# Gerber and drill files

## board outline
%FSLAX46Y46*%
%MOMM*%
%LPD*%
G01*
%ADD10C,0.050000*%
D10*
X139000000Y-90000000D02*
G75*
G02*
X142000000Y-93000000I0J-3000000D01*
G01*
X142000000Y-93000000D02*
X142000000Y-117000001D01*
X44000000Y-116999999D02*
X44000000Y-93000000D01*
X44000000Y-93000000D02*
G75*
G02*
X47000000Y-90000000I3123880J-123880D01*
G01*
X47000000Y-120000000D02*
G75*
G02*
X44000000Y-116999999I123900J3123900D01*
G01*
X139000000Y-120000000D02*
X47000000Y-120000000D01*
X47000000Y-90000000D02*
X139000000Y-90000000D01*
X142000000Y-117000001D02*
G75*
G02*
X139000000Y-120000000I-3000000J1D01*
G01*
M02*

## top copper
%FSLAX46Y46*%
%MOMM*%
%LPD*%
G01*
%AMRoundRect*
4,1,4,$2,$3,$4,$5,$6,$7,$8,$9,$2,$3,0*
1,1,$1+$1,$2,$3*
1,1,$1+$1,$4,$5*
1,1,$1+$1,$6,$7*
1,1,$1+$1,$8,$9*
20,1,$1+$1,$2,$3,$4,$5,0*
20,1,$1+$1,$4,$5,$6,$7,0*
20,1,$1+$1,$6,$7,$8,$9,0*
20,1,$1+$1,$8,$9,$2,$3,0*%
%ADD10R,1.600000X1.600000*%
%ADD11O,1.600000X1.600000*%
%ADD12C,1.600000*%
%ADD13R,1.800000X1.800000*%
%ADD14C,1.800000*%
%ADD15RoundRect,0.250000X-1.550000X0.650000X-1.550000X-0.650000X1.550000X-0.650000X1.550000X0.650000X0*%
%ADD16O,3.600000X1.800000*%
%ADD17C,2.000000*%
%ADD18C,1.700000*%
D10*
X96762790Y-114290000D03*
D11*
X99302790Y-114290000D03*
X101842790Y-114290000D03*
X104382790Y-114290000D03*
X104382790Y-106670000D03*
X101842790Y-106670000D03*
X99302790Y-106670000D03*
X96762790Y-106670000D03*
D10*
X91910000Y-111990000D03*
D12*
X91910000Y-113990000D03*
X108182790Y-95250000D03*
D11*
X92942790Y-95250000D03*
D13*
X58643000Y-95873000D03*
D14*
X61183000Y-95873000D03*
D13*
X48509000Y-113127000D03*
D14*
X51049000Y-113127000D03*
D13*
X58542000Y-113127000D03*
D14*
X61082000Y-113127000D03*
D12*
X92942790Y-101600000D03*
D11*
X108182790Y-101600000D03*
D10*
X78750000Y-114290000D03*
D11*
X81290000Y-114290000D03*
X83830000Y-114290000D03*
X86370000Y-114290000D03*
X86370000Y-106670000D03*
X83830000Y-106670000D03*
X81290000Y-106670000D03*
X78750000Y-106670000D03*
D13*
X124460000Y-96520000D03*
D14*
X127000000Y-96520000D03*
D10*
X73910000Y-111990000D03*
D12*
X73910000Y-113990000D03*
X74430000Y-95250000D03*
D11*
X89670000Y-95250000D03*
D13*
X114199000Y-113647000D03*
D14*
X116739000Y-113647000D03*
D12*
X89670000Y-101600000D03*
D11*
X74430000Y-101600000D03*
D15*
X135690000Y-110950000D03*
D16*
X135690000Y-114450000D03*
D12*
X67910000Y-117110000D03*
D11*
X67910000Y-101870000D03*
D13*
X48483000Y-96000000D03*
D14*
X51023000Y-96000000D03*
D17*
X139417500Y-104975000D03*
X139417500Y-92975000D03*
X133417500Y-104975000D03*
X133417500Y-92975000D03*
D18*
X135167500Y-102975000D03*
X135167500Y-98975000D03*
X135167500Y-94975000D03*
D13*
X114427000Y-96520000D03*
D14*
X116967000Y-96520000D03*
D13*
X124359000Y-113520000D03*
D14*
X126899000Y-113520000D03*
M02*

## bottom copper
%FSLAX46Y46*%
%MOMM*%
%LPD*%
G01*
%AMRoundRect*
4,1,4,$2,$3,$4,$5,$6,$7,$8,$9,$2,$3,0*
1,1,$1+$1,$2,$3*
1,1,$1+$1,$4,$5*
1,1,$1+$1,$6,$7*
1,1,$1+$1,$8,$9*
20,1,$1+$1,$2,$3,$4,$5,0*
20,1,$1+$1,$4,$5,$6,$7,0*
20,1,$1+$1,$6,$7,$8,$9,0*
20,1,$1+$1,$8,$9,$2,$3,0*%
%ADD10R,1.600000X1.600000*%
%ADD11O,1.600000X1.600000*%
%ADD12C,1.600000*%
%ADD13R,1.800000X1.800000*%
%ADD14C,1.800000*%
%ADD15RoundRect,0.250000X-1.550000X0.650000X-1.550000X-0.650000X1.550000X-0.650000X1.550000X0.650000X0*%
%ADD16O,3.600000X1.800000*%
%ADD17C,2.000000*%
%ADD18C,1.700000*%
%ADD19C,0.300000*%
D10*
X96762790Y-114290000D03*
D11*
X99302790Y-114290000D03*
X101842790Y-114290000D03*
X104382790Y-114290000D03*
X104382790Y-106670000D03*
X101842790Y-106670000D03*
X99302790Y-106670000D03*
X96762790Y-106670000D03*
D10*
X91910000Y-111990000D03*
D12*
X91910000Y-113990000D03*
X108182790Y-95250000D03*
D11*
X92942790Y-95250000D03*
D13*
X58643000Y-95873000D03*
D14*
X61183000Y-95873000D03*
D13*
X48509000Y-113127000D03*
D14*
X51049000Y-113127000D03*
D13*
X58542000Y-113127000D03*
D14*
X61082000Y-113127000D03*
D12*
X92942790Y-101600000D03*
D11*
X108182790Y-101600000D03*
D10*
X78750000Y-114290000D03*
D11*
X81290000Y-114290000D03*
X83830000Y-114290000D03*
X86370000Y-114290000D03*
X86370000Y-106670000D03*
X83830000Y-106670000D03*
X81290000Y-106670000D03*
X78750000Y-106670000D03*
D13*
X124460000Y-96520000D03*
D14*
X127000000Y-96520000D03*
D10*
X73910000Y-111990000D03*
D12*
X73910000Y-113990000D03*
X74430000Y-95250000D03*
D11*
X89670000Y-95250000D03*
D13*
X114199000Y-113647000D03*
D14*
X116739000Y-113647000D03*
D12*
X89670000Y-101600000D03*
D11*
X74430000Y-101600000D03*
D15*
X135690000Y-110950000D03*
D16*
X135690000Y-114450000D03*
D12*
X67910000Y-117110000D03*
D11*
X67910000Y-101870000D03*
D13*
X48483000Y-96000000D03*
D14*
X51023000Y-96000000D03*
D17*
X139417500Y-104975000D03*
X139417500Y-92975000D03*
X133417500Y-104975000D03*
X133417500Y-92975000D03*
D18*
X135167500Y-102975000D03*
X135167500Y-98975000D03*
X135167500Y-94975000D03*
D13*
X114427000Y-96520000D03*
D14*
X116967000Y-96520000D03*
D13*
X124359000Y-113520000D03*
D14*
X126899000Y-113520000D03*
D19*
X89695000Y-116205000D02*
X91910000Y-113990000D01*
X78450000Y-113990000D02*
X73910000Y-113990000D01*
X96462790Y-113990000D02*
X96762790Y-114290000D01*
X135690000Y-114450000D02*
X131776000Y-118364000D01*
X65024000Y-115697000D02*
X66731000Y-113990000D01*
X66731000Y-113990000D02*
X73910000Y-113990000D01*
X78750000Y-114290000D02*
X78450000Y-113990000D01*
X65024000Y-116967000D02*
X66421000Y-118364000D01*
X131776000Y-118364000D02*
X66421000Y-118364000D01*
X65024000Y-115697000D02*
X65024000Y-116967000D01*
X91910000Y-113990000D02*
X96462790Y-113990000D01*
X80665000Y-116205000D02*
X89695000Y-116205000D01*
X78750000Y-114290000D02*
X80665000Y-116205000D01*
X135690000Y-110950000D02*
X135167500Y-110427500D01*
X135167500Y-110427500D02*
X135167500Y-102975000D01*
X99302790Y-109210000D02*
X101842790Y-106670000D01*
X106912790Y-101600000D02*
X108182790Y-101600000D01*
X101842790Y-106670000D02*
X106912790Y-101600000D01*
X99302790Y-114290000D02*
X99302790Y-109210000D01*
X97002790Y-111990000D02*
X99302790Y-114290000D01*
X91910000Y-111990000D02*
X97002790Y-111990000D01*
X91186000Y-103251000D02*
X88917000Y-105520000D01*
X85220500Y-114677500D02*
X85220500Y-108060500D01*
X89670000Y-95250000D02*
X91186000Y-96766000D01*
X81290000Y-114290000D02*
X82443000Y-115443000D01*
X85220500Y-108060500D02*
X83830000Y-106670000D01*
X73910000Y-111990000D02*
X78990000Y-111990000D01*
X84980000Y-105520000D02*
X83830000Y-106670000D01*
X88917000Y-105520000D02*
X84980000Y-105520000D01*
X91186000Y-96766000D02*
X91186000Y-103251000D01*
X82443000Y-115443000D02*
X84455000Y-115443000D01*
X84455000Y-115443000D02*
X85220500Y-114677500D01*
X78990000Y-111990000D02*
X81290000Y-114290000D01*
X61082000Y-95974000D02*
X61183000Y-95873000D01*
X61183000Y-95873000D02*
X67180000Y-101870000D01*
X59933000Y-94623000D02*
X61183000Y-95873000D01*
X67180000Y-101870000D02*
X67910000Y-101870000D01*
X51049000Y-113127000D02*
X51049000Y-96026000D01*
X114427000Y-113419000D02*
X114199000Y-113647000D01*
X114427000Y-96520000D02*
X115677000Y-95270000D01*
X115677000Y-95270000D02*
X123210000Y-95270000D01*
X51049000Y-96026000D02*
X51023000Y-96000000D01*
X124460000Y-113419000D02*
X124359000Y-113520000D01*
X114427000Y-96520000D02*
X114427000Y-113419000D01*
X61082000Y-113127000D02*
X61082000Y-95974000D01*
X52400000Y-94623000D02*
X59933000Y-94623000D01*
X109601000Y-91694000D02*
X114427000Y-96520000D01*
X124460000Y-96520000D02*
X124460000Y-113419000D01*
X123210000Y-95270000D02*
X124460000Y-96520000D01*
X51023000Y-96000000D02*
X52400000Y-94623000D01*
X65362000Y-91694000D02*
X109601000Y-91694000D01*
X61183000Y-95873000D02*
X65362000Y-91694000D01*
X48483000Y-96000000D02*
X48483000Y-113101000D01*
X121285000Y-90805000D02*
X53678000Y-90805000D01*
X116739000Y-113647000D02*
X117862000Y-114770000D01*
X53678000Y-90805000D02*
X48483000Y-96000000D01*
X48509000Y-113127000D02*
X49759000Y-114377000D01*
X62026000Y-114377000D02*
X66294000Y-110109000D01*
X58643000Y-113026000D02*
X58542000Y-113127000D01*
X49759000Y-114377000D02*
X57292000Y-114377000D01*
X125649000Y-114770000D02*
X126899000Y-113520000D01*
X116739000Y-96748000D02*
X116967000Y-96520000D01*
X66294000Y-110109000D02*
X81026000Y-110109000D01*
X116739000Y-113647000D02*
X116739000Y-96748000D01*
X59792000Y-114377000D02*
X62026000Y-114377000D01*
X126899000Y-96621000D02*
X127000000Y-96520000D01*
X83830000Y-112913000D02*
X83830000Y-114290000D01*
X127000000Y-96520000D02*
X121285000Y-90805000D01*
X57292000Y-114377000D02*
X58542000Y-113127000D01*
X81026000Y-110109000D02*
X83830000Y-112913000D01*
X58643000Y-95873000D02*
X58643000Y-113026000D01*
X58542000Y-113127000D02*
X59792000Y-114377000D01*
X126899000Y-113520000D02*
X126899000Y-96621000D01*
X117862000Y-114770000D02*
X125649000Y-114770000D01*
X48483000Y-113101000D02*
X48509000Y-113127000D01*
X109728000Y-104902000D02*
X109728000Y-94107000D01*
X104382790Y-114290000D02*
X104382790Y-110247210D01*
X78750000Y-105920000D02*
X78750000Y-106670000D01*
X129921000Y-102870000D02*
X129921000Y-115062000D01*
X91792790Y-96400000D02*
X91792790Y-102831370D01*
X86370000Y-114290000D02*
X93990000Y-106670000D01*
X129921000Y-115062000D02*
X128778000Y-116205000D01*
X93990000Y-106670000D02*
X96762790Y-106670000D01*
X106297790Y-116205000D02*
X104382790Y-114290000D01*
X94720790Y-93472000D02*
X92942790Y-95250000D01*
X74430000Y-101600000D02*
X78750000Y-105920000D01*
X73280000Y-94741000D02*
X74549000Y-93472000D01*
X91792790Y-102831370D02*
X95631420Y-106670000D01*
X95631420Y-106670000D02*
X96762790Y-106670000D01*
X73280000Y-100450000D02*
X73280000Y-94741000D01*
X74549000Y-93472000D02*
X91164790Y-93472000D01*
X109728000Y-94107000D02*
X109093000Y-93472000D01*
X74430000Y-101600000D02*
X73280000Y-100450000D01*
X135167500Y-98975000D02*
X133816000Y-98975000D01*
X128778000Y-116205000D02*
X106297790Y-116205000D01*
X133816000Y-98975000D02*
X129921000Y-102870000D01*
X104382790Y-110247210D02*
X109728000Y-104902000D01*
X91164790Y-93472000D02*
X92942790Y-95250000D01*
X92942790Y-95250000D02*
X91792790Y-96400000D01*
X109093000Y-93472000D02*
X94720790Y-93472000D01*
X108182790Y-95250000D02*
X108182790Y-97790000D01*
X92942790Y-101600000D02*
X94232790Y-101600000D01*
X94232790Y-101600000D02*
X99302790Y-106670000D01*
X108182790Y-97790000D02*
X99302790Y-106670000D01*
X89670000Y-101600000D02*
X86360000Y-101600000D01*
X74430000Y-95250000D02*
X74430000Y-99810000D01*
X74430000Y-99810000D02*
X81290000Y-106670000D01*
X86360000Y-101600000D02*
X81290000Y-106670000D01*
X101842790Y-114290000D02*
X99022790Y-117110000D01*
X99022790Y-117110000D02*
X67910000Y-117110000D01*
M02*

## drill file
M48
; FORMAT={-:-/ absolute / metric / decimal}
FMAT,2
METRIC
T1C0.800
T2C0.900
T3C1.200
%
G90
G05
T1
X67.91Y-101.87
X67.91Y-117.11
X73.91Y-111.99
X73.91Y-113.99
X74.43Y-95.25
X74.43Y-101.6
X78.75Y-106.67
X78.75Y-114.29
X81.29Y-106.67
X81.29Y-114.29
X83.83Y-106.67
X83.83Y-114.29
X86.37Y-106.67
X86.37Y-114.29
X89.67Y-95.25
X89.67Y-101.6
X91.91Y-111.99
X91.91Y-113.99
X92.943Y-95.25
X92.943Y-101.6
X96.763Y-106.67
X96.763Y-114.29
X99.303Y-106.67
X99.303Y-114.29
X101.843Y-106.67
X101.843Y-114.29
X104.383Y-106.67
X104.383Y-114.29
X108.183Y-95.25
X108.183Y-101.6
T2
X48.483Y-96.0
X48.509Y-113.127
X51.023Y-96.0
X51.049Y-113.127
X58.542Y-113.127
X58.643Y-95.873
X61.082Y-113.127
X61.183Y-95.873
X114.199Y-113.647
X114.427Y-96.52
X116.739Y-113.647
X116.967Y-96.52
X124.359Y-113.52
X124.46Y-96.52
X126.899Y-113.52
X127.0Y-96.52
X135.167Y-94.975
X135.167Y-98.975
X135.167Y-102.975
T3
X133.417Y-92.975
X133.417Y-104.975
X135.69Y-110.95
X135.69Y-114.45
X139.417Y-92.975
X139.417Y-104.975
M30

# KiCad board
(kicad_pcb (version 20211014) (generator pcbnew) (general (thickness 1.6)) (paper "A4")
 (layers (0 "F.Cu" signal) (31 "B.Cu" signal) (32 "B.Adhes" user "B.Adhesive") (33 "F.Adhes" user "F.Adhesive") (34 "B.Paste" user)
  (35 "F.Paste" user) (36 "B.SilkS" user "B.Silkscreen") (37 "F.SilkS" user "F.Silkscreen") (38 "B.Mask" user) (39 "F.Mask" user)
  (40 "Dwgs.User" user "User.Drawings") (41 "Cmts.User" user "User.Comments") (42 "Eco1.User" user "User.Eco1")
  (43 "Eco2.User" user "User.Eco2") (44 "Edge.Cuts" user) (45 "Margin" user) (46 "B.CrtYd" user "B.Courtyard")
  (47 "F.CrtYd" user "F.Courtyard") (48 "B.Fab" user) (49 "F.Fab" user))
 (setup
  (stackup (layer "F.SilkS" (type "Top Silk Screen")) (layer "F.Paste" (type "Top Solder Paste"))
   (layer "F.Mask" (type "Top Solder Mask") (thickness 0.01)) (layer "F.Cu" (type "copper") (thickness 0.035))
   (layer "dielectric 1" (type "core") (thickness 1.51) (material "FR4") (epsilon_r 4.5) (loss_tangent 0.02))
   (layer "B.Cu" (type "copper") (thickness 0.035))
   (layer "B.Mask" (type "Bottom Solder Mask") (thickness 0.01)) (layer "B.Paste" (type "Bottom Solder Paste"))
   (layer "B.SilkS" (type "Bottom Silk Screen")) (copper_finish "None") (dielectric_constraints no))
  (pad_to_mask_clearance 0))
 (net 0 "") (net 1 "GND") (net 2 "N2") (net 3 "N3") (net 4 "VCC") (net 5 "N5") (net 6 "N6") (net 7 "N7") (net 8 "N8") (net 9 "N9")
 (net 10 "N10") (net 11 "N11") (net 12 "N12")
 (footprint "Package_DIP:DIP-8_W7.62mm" (layer "F.Cu") (at 96.76279 114.29 90)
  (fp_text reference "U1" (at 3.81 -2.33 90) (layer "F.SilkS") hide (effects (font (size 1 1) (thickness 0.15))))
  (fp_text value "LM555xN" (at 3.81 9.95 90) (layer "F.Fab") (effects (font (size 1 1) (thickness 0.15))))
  (pad "1" thru_hole rect (at 0 0 90) (size 1.6 1.6) (drill 0.8) (layers *.Cu *.Mask) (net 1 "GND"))
  (pad "2" thru_hole oval (at 0 2.54 90) (size 1.6 1.6) (drill 0.8) (layers *.Cu *.Mask) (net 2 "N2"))
  (pad "3" thru_hole oval (at 0 5.08 90) (size 1.6 1.6) (drill 0.8) (layers *.Cu *.Mask) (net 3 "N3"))
  (pad "4" thru_hole oval (at 0 7.62 90) (size 1.6 1.6) (drill 0.8) (layers *.Cu *.Mask) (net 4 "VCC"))
  (pad "5" thru_hole oval (at 7.62 7.62 90) (size 1.6 1.6) (drill 0.8) (layers *.Cu *.Mask) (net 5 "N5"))
  (pad "6" thru_hole oval (at 7.62 5.08 90) (size 1.6 1.6) (drill 0.8) (layers *.Cu *.Mask) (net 2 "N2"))
  (pad "7" thru_hole oval (at 7.62 2.54 90) (size 1.6 1.6) (drill 0.8) (layers *.Cu *.Mask) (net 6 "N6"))
  (pad "8" thru_hole oval (at 7.62 0 90) (size 1.6 1.6) (drill 0.8) (layers *.Cu *.Mask) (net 4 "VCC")))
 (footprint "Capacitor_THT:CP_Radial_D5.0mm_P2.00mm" (layer "F.Cu") (at 91.91 111.99 -90)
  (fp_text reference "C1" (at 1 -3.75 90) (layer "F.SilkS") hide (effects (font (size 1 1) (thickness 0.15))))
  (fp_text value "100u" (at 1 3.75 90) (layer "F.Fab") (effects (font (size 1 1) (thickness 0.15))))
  (pad "1" thru_hole rect (at 0 0 270) (size 1.6 1.6) (drill 0.8) (layers *.Cu *.Mask) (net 2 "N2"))
  (pad "2" thru_hole circle (at 2 0 270) (size 1.6 1.6) (drill 0.8) (layers *.Cu *.Mask) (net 1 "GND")))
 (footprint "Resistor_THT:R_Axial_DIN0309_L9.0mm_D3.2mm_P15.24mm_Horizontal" (layer "F.Cu") (at 108.18279 95.25 180)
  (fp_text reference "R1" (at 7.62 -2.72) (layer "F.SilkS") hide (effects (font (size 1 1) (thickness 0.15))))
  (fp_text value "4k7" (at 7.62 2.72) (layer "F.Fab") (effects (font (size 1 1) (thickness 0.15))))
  (pad "1" thru_hole circle (at 0 0 180) (size 1.6 1.6) (drill 0.8) (layers *.Cu *.Mask) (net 6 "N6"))
  (pad "2" thru_hole oval (at 15.24 0 180) (size 1.6 1.6) (drill 0.8) (layers *.Cu *.Mask) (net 4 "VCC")))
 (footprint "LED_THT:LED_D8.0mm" (layer "F.Cu") (at 58.643 95.873)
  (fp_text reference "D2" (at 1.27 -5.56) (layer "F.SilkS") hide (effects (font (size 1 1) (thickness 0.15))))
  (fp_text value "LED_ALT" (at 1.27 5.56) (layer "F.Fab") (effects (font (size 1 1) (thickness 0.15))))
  (pad "1" thru_hole rect (at 0 0) (size 1.8 1.8) (drill 0.9) (layers *.Cu *.Mask) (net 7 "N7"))
  (pad "2" thru_hole circle (at 2.54 0) (size 1.8 1.8) (drill 0.9) (layers *.Cu *.Mask) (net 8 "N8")))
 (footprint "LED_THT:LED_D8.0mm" (layer "F.Cu") (at 48.509 113.127)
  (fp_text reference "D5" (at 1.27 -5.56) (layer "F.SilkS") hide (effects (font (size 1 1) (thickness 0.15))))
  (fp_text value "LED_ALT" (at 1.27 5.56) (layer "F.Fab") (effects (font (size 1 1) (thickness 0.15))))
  (pad "1" thru_hole rect (at 0 0) (size 1.8 1.8) (drill 0.9) (layers *.Cu *.Mask) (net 7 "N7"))
  (pad "2" thru_hole circle (at 2.54 0) (size 1.8 1.8) (drill 0.9) (layers *.Cu *.Mask) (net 8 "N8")))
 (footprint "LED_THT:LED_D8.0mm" (layer "F.Cu") (at 58.542 113.127)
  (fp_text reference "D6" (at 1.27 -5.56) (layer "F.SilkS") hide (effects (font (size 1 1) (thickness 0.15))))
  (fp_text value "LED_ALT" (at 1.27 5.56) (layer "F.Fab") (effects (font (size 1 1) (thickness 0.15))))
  (pad "1" thru_hole rect (at 0 0) (size 1.8 1.8) (drill 0.9) (layers *.Cu *.Mask) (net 7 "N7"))
  (pad "2" thru_hole circle (at 2.54 0) (size 1.8 1.8) (drill 0.9) (layers *.Cu *.Mask) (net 8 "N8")))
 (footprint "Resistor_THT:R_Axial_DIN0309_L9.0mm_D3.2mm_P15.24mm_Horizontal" (layer "F.Cu") (at 92.94279 101.6)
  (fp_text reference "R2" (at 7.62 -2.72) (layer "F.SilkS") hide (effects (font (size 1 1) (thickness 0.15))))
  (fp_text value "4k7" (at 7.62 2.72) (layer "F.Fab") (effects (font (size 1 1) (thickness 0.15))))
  (pad "1" thru_hole circle (at 0 0) (size 1.6 1.6) (drill 0.8) (layers *.Cu *.Mask) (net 6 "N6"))
  (pad "2" thru_hole oval (at 15.24 0) (size 1.6 1.6) (drill 0.8) (layers *.Cu *.Mask) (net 2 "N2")))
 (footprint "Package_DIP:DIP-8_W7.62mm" (layer "F.Cu") (at 78.75 114.29 90)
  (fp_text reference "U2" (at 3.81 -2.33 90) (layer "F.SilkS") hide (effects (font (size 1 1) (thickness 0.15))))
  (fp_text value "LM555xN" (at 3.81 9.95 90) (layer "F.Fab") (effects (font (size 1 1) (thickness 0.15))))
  (pad "1" thru_hole rect (at 0 0 90) (size 1.6 1.6) (drill 0.8) (layers *.Cu *.Mask) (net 1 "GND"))
  (pad "2" thru_hole oval (at 0 2.54 90) (size 1.6 1.6) (drill 0.8) (layers *.Cu *.Mask) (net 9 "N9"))
  (pad "3" thru_hole oval (at 0 5.08 90) (size 1.6 1.6) (drill 0.8) (layers *.Cu *.Mask) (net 7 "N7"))
  (pad "4" thru_hole oval (at 0 7.62 90) (size 1.6 1.6) (drill 0.8) (layers *.Cu *.Mask) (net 4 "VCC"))
  (pad "5" thru_hole oval (at 7.62 7.62 90) (size 1.6 1.6) (drill 0.8) (layers *.Cu *.Mask) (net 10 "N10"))
  (pad "6" thru_hole oval (at 7.62 5.08 90) (size 1.6 1.6) (drill 0.8) (layers *.Cu *.Mask) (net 9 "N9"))
  (pad "7" thru_hole oval (at 7.62 2.54 90) (size 1.6 1.6) (drill 0.8) (layers *.Cu *.Mask) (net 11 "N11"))
  (pad "8" thru_hole oval (at 7.62 0 90) (size 1.6 1.6) (drill 0.8) (layers *.Cu *.Mask) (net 4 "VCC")))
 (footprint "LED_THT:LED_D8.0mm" (layer "F.Cu") (at 124.46 96.52)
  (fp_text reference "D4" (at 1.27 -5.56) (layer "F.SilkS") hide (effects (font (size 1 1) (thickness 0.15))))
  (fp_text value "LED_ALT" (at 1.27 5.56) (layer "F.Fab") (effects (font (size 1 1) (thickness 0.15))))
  (pad "1" thru_hole rect (at 0 0) (size 1.8 1.8) (drill 0.9) (layers *.Cu *.Mask) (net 8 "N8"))
  (pad "2" thru_hole circle (at 2.54 0) (size 1.8 1.8) (drill 0.9) (layers *.Cu *.Mask) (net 7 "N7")))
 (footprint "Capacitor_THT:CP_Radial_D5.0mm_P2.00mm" (layer "F.Cu") (at 73.91 111.99 -90)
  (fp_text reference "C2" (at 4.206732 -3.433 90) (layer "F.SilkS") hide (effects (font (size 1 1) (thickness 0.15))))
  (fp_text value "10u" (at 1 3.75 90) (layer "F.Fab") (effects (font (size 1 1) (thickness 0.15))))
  (pad "1" thru_hole rect (at 0 0 270) (size 1.6 1.6) (drill 0.8) (layers *.Cu *.Mask) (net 9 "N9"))
  (pad "2" thru_hole circle (at 2 0 270) (size 1.6 1.6) (drill 0.8) (layers *.Cu *.Mask) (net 1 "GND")))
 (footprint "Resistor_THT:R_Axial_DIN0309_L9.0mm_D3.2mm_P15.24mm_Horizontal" (layer "F.Cu") (at 74.43 95.25)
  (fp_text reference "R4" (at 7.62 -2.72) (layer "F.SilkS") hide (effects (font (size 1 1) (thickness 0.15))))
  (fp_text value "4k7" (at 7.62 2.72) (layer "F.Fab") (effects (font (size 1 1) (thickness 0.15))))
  (pad "1" thru_hole circle (at 0 0) (size 1.6 1.6) (drill 0.8) (layers *.Cu *.Mask) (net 11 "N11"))
  (pad "2" thru_hole oval (at 15.24 0) (size 1.6 1.6) (drill 0.8) (layers *.Cu *.Mask) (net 9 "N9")))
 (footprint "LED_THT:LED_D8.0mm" (layer "F.Cu") (at 114.199 113.647)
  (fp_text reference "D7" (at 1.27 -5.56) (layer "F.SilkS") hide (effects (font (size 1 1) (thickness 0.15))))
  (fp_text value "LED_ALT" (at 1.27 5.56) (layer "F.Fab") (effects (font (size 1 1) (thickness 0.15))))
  (pad "1" thru_hole rect (at 0 0) (size 1.8 1.8) (drill 0.9) (layers *.Cu *.Mask) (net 8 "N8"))
  (pad "2" thru_hole circle (at 2.54 0) (size 1.8 1.8) (drill 0.9) (layers *.Cu *.Mask) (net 7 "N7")))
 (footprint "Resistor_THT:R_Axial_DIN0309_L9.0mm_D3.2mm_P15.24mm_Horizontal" (layer "F.Cu") (at 89.67 101.6 180)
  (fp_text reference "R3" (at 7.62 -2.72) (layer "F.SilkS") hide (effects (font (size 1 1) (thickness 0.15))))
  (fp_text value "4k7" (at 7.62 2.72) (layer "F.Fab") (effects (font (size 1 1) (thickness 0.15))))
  (pad "1" thru_hole circle (at 0 0 180) (size 1.6 1.6) (drill 0.8) (layers *.Cu *.Mask) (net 11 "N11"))
  (pad "2" thru_hole oval (at 15.24 0 180) (size 1.6 1.6) (drill 0.8) (layers *.Cu *.Mask) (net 4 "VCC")))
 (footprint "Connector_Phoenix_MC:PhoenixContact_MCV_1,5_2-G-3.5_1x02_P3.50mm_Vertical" (layer "F.Cu") (at 135.69 110.95 -90)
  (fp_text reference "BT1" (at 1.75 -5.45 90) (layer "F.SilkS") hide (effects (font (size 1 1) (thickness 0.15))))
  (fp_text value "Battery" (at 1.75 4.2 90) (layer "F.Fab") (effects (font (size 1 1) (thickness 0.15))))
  (pad "1" thru_hole roundrect (at 0 0 270) (size 1.8 3.6) (drill 1.2) (layers *.Cu *.Mask) (roundrect_rratio 0.138889) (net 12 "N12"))
  (pad "2" thru_hole oval (at 3.5 0 270) (size 1.8 3.6) (drill 1.2) (layers *.Cu *.Mask) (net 1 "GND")))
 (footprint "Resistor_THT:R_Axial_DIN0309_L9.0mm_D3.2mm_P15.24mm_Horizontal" (layer "F.Cu") (at 67.91 117.11 90)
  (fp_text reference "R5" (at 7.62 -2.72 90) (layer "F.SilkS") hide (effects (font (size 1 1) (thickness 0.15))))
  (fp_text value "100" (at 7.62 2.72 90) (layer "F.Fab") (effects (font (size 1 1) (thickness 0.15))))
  (pad "1" thru_hole circle (at 0 0 90) (size 1.6 1.6) (drill 0.8) (layers *.Cu *.Mask) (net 3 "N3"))
  (pad "2" thru_hole oval (at 15.24 0 90) (size 1.6 1.6) (drill 0.8) (layers *.Cu *.Mask) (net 8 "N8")))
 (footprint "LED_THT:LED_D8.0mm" (layer "F.Cu") (at 48.483 96)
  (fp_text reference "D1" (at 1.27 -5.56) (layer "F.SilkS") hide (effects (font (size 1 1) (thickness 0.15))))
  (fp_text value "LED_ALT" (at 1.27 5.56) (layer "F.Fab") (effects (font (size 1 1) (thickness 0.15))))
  (pad "1" thru_hole rect (at 0 0) (size 1.8 1.8) (drill 0.9) (layers *.Cu *.Mask) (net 7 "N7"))
  (pad "2" thru_hole circle (at 2.54 0) (size 1.8 1.8) (drill 0.9) (layers *.Cu *.Mask) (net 8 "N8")))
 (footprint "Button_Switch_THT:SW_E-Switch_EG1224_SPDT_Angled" (layer "F.Cu") (at 135.1675 102.975 90)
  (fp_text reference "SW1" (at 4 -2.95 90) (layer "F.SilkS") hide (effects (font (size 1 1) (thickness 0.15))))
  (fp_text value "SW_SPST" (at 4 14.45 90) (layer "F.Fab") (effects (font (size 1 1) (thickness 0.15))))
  (pad "" thru_hole circle (at -2 4.25 90) (size 2 2) (drill 1.2) (layers *.Cu *.Mask))
  (pad "" thru_hole circle (at 10 4.25 90) (size 2 2) (drill 1.2) (layers *.Cu *.Mask))
  (pad "" thru_hole circle (at -2 -1.75 90) (size 2 2) (drill 1.2) (layers *.Cu *.Mask))
  (pad "" thru_hole circle (at 10 -1.75 90) (size 2 2) (drill 1.2) (layers *.Cu *.Mask))
  (pad "1" thru_hole circle (at 0 0 90) (size 1.7 1.7) (drill 0.9) (layers *.Cu *.Mask) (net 12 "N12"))
  (pad "2" thru_hole circle (at 4 0 90) (size 1.7 1.7) (drill 0.9) (layers *.Cu *.Mask) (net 4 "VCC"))
  (pad "3" thru_hole circle (at 8 0 90) (size 1.7 1.7) (drill 0.9) (layers *.Cu *.Mask)))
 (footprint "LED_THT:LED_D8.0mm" (layer "F.Cu") (at 114.427 96.52)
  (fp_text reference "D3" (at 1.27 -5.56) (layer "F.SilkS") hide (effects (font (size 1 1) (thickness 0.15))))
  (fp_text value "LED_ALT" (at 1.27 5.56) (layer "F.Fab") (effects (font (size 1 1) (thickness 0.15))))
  (pad "1" thru_hole rect (at 0 0) (size 1.8 1.8) (drill 0.9) (layers *.Cu *.Mask) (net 8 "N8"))
  (pad "2" thru_hole circle (at 2.54 0) (size 1.8 1.8) (drill 0.9) (layers *.Cu *.Mask) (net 7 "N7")))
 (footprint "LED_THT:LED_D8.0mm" (layer "F.Cu") (at 124.359 113.52)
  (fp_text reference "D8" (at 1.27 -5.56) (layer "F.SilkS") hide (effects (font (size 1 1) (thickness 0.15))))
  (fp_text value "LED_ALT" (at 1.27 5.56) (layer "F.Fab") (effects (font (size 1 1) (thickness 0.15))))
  (pad "1" thru_hole rect (at 0 0) (size 1.8 1.8) (drill 0.9) (layers *.Cu *.Mask) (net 8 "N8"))
  (pad "2" thru_hole circle (at 2.54 0) (size 1.8 1.8) (drill 0.9) (layers *.Cu *.Mask) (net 7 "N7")))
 (gr_arc (start 139 90) (mid 141.12132 90.87868) (end 142 93) (layer "Edge.Cuts") (width 0.05))
 (gr_line (start 142 93) (end 142 117.000001) (layer "Edge.Cuts") (width 0.05))
 (gr_line (start 44 116.999999) (end 44 93) (layer "Edge.Cuts") (width 0.05))
 (gr_arc (start 44 93) (mid 44.913226 90.913226) (end 47 90) (layer "Edge.Cuts") (width 0.05))
 (gr_arc (start 47 120) (mid 44.913226 119.086773) (end 44 116.999999) (layer "Edge.Cuts") (width 0.05))
 (gr_line (start 139 120) (end 47 120) (layer "Edge.Cuts") (width 0.05))
 (gr_line (start 47 90) (end 139 90) (layer "Edge.Cuts") (width 0.05))
 (gr_arc (start 142 117.000001) (mid 141.121318 119.121318) (end 139 120) (layer "Edge.Cuts") (width 0.05))
 (segment (start 89.695 116.205) (end 91.91 113.99) (width 0.3) (layer "B.Cu") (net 1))
 (segment (start 78.45 113.99) (end 73.91 113.99) (width 0.3) (layer "B.Cu") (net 1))
 (segment (start 96.46279 113.99) (end 96.76279 114.29) (width 0.3) (layer "B.Cu") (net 1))
 (segment (start 135.69 114.45) (end 131.776 118.364) (width 0.3) (layer "B.Cu") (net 1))
 (segment (start 65.024 115.697) (end 66.731 113.99) (width 0.3) (layer "B.Cu") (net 1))
 (segment (start 66.731 113.99) (end 73.91 113.99) (width 0.3) (layer "B.Cu") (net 1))
 (segment (start 78.75 114.29) (end 78.45 113.99) (width 0.3) (layer "B.Cu") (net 1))
 (segment (start 65.024 116.967) (end 66.421 118.364) (width 0.3) (layer "B.Cu") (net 1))
 (segment (start 131.776 118.364) (end 66.421 118.364) (width 0.3) (layer "B.Cu") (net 1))
 (segment (start 65.024 115.697) (end 65.024 116.967) (width 0.3) (layer "B.Cu") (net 1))
 (segment (start 91.91 113.99) (end 96.46279 113.99) (width 0.3) (layer "B.Cu") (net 1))
 (segment (start 80.665 116.205) (end 89.695 116.205) (width 0.3) (layer "B.Cu") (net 1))
 (segment (start 78.75 114.29) (end 80.665 116.205) (width 0.3) (layer "B.Cu") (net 1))
 (segment (start 135.69 110.95) (end 135.1675 110.4275) (width 0.3) (layer "B.Cu") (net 12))
 (segment (start 135.1675 110.4275) (end 135.1675 102.975) (width 0.3) (layer "B.Cu") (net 12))
 (segment (start 99.30279 109.21) (end 101.84279 106.67) (width 0.3) (layer "B.Cu") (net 2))
 (segment (start 106.91279 101.6) (end 108.18279 101.6) (width 0.3) (layer "B.Cu") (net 2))
 (segment (start 101.84279 106.67) (end 106.91279 101.6) (width 0.3) (layer "B.Cu") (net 2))
 (segment (start 99.30279 114.29) (end 99.30279 109.21) (width 0.3) (layer "B.Cu") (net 2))
 (segment (start 97.00279 111.99) (end 99.30279 114.29) (width 0.3) (layer "B.Cu") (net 2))
 (segment (start 91.91 111.99) (end 97.00279 111.99) (width 0.3) (layer "B.Cu") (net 2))
 (segment (start 91.186 103.251) (end 88.917 105.52) (width 0.3) (layer "B.Cu") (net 9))
 (segment (start 85.2205 114.6775) (end 85.2205 108.0605) (width 0.3) (layer "B.Cu") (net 9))
 (segment (start 89.67 95.25) (end 91.186 96.766) (width 0.3) (layer "B.Cu") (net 9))
 (segment (start 81.29 114.29) (end 82.443 115.443) (width 0.3) (layer "B.Cu") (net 9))
 (segment (start 85.2205 108.0605) (end 83.83 106.67) (width 0.3) (layer "B.Cu") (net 9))
 (segment (start 73.91 111.99) (end 78.99 111.99) (width 0.3) (layer "B.Cu") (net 9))
 (segment (start 84.98 105.52) (end 83.83 106.67) (width 0.3) (layer "B.Cu") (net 9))
 (segment (start 88.917 105.52) (end 84.98 105.52) (width 0.3) (layer "B.Cu") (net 9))
 (segment (start 91.186 96.766) (end 91.186 103.251) (width 0.3) (layer "B.Cu") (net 9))
 (segment (start 82.443 115.443) (end 84.455 115.443) (width 0.3) (layer "B.Cu") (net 9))
 (segment (start 84.455 115.443) (end 85.2205 114.6775) (width 0.3) (layer "B.Cu") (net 9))
 (segment (start 78.99 111.99) (end 81.29 114.29) (width 0.3) (layer "B.Cu") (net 9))
 (segment (start 61.082 95.974) (end 61.183 95.873) (width 0.3) (layer "B.Cu") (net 8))
 (segment (start 61.183 95.873) (end 67.18 101.87) (width 0.3) (layer "B.Cu") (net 8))
 (segment (start 59.933 94.623) (end 61.183 95.873) (width 0.3) (layer "B.Cu") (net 8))
 (segment (start 67.18 101.87) (end 67.91 101.87) (width 0.3) (layer "B.Cu") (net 8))
 (segment (start 51.049 113.127) (end 51.049 96.026) (width 0.3) (layer "B.Cu") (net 8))
 (segment (start 114.427 113.419) (end 114.199 113.647) (width 0.3) (layer "B.Cu") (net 8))
 (segment (start 114.427 96.52) (end 115.677 95.27) (width 0.3) (layer "B.Cu") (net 8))
 (segment (start 115.677 95.27) (end 123.21 95.27) (width 0.3) (layer "B.Cu") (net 8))
 (segment (start 51.049 96.026) (end 51.023 96) (width 0.3) (layer "B.Cu") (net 8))
 (segment (start 124.46 113.419) (end 124.359 113.52) (width 0.3) (layer "B.Cu") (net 8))
 (segment (start 114.427 96.52) (end 114.427 113.419) (width 0.3) (layer "B.Cu") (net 8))
 (segment (start 61.082 113.127) (end 61.082 95.974) (width 0.3) (layer "B.Cu") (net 8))
 (segment (start 52.4 94.623) (end 59.933 94.623) (width 0.3) (layer "B.Cu") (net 8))
 (segment (start 109.601 91.694) (end 114.427 96.52) (width 0.3) (layer "B.Cu") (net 8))
 (segment (start 124.46 96.52) (end 124.46 113.419) (width 0.3) (layer "B.Cu") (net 8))
 (segment (start 123.21 95.27) (end 124.46 96.52) (width 0.3) (layer "B.Cu") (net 8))
 (segment (start 51.023 96) (end 52.4 94.623) (width 0.3) (layer "B.Cu") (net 8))
 (segment (start 65.362 91.694) (end 109.601 91.694) (width 0.3) (layer "B.Cu") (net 8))
 (segment (start 61.183 95.873) (end 65.362 91.694) (width 0.3) (layer "B.Cu") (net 8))
 (segment (start 48.483 96) (end 48.483 113.101) (width 0.3) (layer "B.Cu") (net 7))
 (segment (start 121.285 90.805) (end 53.678 90.805) (width 0.3) (layer "B.Cu") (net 7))
 (segment (start 116.739 113.647) (end 117.862 114.77) (width 0.3) (layer "B.Cu") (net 7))
 (segment (start 53.678 90.805) (end 48.483 96) (width 0.3) (layer "B.Cu") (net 7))
 (segment (start 48.509 113.127) (end 49.759 114.377) (width 0.3) (layer "B.Cu") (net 7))
 (segment (start 62.026 114.377) (end 66.294 110.109) (width 0.3) (layer "B.Cu") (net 7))
 (segment (start 58.643 113.026) (end 58.542 113.127) (width 0.3) (layer "B.Cu") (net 7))
 (segment (start 49.759 114.377) (end 57.292 114.377) (width 0.3) (layer "B.Cu") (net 7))
 (segment (start 125.649 114.77) (end 126.899 113.52) (width 0.3) (layer "B.Cu") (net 7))
 (segment (start 116.739 96.748) (end 116.967 96.52) (width 0.3) (layer "B.Cu") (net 7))
 (segment (start 66.294 110.109) (end 81.026 110.109) (width 0.3) (layer "B.Cu") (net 7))
 (segment (start 116.739 113.647) (end 116.739 96.748) (width 0.3) (layer "B.Cu") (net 7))
 (segment (start 59.792 114.377) (end 62.026 114.377) (width 0.3) (layer "B.Cu") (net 7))
 (segment (start 126.899 96.621) (end 127 96.52) (width 0.3) (layer "B.Cu") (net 7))
 (segment (start 83.83 112.913) (end 83.83 114.29) (width 0.3) (layer "B.Cu") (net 7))
 (segment (start 127 96.52) (end 121.285 90.805) (width 0.3) (layer "B.Cu") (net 7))
 (segment (start 57.292 114.377) (end 58.542 113.127) (width 0.3) (layer "B.Cu") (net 7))
 (segment (start 81.026 110.109) (end 83.83 112.913) (width 0.3) (layer "B.Cu") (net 7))
 (segment (start 58.643 95.873) (end 58.643 113.026) (width 0.3) (layer "B.Cu") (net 7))
 (segment (start 58.542 113.127) (end 59.792 114.377) (width 0.3) (layer "B.Cu") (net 7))
 (segment (start 126.899 113.52) (end 126.899 96.621) (width 0.3) (layer "B.Cu") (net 7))
 (segment (start 117.862 114.77) (end 125.649 114.77) (width 0.3) (layer "B.Cu") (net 7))
 (segment (start 48.483 113.101) (end 48.509 113.127) (width 0.3) (layer "B.Cu") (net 7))
 (segment (start 109.728 104.902) (end 109.728 94.107) (width 0.3) (layer "B.Cu") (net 4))
 (segment (start 104.38279 114.29) (end 104.38279 110.24721) (width 0.3) (layer "B.Cu") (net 4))
 (segment (start 78.75 105.92) (end 78.75 106.67) (width 0.3) (layer "B.Cu") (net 4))
 (segment (start 129.921 102.87) (end 129.921 115.062) (width 0.3) (layer "B.Cu") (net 4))
 (segment (start 91.79279 96.4) (end 91.79279 102.83137) (width 0.3) (layer "B.Cu") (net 4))
 (segment (start 86.37 114.29) (end 93.99 106.67) (width 0.3) (layer "B.Cu") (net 4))
 (segment (start 129.921 115.062) (end 128.778 116.205) (width 0.3) (layer "B.Cu") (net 4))
 (segment (start 93.99 106.67) (end 96.76279 106.67) (width 0.3) (layer "B.Cu") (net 4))
 (segment (start 106.29779 116.205) (end 104.38279 114.29) (width 0.3) (layer "B.Cu") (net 4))
 (segment (start 94.72079 93.472) (end 92.94279 95.25) (width 0.3) (layer "B.Cu") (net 4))
 (segment (start 74.43 101.6) (end 78.75 105.92) (width 0.3) (layer "B.Cu") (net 4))
 (segment (start 73.28 94.741) (end 74.549 93.472) (width 0.3) (layer "B.Cu") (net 4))
 (segment (start 91.79279 102.83137) (end 95.63142 106.67) (width 0.3) (layer "B.Cu") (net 4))
 (segment (start 95.63142 106.67) (end 96.76279 106.67) (width 0.3) (layer "B.Cu") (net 4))
 (segment (start 73.28 100.45) (end 73.28 94.741) (width 0.3) (layer "B.Cu") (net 4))
 (segment (start 74.549 93.472) (end 91.16479 93.472) (width 0.3) (layer "B.Cu") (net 4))
 (segment (start 109.728 94.107) (end 109.093 93.472) (width 0.3) (layer "B.Cu") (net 4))
 (segment (start 74.43 101.6) (end 73.28 100.45) (width 0.3) (layer "B.Cu") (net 4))
 (segment (start 135.1675 98.975) (end 133.816 98.975) (width 0.3) (layer "B.Cu") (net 4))
 (segment (start 128.778 116.205) (end 106.29779 116.205) (width 0.3) (layer "B.Cu") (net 4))
 (segment (start 133.816 98.975) (end 129.921 102.87) (width 0.3) (layer "B.Cu") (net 4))
 (segment (start 104.38279 110.24721) (end 109.728 104.902) (width 0.3) (layer "B.Cu") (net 4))
 (segment (start 91.16479 93.472) (end 92.94279 95.25) (width 0.3) (layer "B.Cu") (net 4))
 (segment (start 92.94279 95.25) (end 91.79279 96.4) (width 0.3) (layer "B.Cu") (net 4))
 (segment (start 109.093 93.472) (end 94.72079 93.472) (width 0.3) (layer "B.Cu") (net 4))
 (segment (start 108.18279 95.25) (end 108.18279 97.79) (width 0.3) (layer "B.Cu") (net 6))
 (segment (start 92.94279 101.6) (end 94.23279 101.6) (width 0.3) (layer "B.Cu") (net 6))
 (segment (start 94.23279 101.6) (end 99.30279 106.67) (width 0.3) (layer "B.Cu") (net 6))
 (segment (start 108.18279 97.79) (end 99.30279 106.67) (width 0.3) (layer "B.Cu") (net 6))
 (segment (start 89.67 101.6) (end 86.36 101.6) (width 0.3) (layer "B.Cu") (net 11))
 (segment (start 74.43 95.25) (end 74.43 99.81) (width 0.3) (layer "B.Cu") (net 11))
 (segment (start 74.43 99.81) (end 81.29 106.67) (width 0.3) (layer "B.Cu") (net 11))
 (segment (start 86.36 101.6) (end 81.29 106.67) (width 0.3) (layer "B.Cu") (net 11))
 (segment (start 101.84279 114.29) (end 99.02279 117.11) (width 0.3) (layer "B.Cu") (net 3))
 (segment (start 99.02279 117.11) (end 67.91 117.11) (width 0.3) (layer "B.Cu") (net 3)))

